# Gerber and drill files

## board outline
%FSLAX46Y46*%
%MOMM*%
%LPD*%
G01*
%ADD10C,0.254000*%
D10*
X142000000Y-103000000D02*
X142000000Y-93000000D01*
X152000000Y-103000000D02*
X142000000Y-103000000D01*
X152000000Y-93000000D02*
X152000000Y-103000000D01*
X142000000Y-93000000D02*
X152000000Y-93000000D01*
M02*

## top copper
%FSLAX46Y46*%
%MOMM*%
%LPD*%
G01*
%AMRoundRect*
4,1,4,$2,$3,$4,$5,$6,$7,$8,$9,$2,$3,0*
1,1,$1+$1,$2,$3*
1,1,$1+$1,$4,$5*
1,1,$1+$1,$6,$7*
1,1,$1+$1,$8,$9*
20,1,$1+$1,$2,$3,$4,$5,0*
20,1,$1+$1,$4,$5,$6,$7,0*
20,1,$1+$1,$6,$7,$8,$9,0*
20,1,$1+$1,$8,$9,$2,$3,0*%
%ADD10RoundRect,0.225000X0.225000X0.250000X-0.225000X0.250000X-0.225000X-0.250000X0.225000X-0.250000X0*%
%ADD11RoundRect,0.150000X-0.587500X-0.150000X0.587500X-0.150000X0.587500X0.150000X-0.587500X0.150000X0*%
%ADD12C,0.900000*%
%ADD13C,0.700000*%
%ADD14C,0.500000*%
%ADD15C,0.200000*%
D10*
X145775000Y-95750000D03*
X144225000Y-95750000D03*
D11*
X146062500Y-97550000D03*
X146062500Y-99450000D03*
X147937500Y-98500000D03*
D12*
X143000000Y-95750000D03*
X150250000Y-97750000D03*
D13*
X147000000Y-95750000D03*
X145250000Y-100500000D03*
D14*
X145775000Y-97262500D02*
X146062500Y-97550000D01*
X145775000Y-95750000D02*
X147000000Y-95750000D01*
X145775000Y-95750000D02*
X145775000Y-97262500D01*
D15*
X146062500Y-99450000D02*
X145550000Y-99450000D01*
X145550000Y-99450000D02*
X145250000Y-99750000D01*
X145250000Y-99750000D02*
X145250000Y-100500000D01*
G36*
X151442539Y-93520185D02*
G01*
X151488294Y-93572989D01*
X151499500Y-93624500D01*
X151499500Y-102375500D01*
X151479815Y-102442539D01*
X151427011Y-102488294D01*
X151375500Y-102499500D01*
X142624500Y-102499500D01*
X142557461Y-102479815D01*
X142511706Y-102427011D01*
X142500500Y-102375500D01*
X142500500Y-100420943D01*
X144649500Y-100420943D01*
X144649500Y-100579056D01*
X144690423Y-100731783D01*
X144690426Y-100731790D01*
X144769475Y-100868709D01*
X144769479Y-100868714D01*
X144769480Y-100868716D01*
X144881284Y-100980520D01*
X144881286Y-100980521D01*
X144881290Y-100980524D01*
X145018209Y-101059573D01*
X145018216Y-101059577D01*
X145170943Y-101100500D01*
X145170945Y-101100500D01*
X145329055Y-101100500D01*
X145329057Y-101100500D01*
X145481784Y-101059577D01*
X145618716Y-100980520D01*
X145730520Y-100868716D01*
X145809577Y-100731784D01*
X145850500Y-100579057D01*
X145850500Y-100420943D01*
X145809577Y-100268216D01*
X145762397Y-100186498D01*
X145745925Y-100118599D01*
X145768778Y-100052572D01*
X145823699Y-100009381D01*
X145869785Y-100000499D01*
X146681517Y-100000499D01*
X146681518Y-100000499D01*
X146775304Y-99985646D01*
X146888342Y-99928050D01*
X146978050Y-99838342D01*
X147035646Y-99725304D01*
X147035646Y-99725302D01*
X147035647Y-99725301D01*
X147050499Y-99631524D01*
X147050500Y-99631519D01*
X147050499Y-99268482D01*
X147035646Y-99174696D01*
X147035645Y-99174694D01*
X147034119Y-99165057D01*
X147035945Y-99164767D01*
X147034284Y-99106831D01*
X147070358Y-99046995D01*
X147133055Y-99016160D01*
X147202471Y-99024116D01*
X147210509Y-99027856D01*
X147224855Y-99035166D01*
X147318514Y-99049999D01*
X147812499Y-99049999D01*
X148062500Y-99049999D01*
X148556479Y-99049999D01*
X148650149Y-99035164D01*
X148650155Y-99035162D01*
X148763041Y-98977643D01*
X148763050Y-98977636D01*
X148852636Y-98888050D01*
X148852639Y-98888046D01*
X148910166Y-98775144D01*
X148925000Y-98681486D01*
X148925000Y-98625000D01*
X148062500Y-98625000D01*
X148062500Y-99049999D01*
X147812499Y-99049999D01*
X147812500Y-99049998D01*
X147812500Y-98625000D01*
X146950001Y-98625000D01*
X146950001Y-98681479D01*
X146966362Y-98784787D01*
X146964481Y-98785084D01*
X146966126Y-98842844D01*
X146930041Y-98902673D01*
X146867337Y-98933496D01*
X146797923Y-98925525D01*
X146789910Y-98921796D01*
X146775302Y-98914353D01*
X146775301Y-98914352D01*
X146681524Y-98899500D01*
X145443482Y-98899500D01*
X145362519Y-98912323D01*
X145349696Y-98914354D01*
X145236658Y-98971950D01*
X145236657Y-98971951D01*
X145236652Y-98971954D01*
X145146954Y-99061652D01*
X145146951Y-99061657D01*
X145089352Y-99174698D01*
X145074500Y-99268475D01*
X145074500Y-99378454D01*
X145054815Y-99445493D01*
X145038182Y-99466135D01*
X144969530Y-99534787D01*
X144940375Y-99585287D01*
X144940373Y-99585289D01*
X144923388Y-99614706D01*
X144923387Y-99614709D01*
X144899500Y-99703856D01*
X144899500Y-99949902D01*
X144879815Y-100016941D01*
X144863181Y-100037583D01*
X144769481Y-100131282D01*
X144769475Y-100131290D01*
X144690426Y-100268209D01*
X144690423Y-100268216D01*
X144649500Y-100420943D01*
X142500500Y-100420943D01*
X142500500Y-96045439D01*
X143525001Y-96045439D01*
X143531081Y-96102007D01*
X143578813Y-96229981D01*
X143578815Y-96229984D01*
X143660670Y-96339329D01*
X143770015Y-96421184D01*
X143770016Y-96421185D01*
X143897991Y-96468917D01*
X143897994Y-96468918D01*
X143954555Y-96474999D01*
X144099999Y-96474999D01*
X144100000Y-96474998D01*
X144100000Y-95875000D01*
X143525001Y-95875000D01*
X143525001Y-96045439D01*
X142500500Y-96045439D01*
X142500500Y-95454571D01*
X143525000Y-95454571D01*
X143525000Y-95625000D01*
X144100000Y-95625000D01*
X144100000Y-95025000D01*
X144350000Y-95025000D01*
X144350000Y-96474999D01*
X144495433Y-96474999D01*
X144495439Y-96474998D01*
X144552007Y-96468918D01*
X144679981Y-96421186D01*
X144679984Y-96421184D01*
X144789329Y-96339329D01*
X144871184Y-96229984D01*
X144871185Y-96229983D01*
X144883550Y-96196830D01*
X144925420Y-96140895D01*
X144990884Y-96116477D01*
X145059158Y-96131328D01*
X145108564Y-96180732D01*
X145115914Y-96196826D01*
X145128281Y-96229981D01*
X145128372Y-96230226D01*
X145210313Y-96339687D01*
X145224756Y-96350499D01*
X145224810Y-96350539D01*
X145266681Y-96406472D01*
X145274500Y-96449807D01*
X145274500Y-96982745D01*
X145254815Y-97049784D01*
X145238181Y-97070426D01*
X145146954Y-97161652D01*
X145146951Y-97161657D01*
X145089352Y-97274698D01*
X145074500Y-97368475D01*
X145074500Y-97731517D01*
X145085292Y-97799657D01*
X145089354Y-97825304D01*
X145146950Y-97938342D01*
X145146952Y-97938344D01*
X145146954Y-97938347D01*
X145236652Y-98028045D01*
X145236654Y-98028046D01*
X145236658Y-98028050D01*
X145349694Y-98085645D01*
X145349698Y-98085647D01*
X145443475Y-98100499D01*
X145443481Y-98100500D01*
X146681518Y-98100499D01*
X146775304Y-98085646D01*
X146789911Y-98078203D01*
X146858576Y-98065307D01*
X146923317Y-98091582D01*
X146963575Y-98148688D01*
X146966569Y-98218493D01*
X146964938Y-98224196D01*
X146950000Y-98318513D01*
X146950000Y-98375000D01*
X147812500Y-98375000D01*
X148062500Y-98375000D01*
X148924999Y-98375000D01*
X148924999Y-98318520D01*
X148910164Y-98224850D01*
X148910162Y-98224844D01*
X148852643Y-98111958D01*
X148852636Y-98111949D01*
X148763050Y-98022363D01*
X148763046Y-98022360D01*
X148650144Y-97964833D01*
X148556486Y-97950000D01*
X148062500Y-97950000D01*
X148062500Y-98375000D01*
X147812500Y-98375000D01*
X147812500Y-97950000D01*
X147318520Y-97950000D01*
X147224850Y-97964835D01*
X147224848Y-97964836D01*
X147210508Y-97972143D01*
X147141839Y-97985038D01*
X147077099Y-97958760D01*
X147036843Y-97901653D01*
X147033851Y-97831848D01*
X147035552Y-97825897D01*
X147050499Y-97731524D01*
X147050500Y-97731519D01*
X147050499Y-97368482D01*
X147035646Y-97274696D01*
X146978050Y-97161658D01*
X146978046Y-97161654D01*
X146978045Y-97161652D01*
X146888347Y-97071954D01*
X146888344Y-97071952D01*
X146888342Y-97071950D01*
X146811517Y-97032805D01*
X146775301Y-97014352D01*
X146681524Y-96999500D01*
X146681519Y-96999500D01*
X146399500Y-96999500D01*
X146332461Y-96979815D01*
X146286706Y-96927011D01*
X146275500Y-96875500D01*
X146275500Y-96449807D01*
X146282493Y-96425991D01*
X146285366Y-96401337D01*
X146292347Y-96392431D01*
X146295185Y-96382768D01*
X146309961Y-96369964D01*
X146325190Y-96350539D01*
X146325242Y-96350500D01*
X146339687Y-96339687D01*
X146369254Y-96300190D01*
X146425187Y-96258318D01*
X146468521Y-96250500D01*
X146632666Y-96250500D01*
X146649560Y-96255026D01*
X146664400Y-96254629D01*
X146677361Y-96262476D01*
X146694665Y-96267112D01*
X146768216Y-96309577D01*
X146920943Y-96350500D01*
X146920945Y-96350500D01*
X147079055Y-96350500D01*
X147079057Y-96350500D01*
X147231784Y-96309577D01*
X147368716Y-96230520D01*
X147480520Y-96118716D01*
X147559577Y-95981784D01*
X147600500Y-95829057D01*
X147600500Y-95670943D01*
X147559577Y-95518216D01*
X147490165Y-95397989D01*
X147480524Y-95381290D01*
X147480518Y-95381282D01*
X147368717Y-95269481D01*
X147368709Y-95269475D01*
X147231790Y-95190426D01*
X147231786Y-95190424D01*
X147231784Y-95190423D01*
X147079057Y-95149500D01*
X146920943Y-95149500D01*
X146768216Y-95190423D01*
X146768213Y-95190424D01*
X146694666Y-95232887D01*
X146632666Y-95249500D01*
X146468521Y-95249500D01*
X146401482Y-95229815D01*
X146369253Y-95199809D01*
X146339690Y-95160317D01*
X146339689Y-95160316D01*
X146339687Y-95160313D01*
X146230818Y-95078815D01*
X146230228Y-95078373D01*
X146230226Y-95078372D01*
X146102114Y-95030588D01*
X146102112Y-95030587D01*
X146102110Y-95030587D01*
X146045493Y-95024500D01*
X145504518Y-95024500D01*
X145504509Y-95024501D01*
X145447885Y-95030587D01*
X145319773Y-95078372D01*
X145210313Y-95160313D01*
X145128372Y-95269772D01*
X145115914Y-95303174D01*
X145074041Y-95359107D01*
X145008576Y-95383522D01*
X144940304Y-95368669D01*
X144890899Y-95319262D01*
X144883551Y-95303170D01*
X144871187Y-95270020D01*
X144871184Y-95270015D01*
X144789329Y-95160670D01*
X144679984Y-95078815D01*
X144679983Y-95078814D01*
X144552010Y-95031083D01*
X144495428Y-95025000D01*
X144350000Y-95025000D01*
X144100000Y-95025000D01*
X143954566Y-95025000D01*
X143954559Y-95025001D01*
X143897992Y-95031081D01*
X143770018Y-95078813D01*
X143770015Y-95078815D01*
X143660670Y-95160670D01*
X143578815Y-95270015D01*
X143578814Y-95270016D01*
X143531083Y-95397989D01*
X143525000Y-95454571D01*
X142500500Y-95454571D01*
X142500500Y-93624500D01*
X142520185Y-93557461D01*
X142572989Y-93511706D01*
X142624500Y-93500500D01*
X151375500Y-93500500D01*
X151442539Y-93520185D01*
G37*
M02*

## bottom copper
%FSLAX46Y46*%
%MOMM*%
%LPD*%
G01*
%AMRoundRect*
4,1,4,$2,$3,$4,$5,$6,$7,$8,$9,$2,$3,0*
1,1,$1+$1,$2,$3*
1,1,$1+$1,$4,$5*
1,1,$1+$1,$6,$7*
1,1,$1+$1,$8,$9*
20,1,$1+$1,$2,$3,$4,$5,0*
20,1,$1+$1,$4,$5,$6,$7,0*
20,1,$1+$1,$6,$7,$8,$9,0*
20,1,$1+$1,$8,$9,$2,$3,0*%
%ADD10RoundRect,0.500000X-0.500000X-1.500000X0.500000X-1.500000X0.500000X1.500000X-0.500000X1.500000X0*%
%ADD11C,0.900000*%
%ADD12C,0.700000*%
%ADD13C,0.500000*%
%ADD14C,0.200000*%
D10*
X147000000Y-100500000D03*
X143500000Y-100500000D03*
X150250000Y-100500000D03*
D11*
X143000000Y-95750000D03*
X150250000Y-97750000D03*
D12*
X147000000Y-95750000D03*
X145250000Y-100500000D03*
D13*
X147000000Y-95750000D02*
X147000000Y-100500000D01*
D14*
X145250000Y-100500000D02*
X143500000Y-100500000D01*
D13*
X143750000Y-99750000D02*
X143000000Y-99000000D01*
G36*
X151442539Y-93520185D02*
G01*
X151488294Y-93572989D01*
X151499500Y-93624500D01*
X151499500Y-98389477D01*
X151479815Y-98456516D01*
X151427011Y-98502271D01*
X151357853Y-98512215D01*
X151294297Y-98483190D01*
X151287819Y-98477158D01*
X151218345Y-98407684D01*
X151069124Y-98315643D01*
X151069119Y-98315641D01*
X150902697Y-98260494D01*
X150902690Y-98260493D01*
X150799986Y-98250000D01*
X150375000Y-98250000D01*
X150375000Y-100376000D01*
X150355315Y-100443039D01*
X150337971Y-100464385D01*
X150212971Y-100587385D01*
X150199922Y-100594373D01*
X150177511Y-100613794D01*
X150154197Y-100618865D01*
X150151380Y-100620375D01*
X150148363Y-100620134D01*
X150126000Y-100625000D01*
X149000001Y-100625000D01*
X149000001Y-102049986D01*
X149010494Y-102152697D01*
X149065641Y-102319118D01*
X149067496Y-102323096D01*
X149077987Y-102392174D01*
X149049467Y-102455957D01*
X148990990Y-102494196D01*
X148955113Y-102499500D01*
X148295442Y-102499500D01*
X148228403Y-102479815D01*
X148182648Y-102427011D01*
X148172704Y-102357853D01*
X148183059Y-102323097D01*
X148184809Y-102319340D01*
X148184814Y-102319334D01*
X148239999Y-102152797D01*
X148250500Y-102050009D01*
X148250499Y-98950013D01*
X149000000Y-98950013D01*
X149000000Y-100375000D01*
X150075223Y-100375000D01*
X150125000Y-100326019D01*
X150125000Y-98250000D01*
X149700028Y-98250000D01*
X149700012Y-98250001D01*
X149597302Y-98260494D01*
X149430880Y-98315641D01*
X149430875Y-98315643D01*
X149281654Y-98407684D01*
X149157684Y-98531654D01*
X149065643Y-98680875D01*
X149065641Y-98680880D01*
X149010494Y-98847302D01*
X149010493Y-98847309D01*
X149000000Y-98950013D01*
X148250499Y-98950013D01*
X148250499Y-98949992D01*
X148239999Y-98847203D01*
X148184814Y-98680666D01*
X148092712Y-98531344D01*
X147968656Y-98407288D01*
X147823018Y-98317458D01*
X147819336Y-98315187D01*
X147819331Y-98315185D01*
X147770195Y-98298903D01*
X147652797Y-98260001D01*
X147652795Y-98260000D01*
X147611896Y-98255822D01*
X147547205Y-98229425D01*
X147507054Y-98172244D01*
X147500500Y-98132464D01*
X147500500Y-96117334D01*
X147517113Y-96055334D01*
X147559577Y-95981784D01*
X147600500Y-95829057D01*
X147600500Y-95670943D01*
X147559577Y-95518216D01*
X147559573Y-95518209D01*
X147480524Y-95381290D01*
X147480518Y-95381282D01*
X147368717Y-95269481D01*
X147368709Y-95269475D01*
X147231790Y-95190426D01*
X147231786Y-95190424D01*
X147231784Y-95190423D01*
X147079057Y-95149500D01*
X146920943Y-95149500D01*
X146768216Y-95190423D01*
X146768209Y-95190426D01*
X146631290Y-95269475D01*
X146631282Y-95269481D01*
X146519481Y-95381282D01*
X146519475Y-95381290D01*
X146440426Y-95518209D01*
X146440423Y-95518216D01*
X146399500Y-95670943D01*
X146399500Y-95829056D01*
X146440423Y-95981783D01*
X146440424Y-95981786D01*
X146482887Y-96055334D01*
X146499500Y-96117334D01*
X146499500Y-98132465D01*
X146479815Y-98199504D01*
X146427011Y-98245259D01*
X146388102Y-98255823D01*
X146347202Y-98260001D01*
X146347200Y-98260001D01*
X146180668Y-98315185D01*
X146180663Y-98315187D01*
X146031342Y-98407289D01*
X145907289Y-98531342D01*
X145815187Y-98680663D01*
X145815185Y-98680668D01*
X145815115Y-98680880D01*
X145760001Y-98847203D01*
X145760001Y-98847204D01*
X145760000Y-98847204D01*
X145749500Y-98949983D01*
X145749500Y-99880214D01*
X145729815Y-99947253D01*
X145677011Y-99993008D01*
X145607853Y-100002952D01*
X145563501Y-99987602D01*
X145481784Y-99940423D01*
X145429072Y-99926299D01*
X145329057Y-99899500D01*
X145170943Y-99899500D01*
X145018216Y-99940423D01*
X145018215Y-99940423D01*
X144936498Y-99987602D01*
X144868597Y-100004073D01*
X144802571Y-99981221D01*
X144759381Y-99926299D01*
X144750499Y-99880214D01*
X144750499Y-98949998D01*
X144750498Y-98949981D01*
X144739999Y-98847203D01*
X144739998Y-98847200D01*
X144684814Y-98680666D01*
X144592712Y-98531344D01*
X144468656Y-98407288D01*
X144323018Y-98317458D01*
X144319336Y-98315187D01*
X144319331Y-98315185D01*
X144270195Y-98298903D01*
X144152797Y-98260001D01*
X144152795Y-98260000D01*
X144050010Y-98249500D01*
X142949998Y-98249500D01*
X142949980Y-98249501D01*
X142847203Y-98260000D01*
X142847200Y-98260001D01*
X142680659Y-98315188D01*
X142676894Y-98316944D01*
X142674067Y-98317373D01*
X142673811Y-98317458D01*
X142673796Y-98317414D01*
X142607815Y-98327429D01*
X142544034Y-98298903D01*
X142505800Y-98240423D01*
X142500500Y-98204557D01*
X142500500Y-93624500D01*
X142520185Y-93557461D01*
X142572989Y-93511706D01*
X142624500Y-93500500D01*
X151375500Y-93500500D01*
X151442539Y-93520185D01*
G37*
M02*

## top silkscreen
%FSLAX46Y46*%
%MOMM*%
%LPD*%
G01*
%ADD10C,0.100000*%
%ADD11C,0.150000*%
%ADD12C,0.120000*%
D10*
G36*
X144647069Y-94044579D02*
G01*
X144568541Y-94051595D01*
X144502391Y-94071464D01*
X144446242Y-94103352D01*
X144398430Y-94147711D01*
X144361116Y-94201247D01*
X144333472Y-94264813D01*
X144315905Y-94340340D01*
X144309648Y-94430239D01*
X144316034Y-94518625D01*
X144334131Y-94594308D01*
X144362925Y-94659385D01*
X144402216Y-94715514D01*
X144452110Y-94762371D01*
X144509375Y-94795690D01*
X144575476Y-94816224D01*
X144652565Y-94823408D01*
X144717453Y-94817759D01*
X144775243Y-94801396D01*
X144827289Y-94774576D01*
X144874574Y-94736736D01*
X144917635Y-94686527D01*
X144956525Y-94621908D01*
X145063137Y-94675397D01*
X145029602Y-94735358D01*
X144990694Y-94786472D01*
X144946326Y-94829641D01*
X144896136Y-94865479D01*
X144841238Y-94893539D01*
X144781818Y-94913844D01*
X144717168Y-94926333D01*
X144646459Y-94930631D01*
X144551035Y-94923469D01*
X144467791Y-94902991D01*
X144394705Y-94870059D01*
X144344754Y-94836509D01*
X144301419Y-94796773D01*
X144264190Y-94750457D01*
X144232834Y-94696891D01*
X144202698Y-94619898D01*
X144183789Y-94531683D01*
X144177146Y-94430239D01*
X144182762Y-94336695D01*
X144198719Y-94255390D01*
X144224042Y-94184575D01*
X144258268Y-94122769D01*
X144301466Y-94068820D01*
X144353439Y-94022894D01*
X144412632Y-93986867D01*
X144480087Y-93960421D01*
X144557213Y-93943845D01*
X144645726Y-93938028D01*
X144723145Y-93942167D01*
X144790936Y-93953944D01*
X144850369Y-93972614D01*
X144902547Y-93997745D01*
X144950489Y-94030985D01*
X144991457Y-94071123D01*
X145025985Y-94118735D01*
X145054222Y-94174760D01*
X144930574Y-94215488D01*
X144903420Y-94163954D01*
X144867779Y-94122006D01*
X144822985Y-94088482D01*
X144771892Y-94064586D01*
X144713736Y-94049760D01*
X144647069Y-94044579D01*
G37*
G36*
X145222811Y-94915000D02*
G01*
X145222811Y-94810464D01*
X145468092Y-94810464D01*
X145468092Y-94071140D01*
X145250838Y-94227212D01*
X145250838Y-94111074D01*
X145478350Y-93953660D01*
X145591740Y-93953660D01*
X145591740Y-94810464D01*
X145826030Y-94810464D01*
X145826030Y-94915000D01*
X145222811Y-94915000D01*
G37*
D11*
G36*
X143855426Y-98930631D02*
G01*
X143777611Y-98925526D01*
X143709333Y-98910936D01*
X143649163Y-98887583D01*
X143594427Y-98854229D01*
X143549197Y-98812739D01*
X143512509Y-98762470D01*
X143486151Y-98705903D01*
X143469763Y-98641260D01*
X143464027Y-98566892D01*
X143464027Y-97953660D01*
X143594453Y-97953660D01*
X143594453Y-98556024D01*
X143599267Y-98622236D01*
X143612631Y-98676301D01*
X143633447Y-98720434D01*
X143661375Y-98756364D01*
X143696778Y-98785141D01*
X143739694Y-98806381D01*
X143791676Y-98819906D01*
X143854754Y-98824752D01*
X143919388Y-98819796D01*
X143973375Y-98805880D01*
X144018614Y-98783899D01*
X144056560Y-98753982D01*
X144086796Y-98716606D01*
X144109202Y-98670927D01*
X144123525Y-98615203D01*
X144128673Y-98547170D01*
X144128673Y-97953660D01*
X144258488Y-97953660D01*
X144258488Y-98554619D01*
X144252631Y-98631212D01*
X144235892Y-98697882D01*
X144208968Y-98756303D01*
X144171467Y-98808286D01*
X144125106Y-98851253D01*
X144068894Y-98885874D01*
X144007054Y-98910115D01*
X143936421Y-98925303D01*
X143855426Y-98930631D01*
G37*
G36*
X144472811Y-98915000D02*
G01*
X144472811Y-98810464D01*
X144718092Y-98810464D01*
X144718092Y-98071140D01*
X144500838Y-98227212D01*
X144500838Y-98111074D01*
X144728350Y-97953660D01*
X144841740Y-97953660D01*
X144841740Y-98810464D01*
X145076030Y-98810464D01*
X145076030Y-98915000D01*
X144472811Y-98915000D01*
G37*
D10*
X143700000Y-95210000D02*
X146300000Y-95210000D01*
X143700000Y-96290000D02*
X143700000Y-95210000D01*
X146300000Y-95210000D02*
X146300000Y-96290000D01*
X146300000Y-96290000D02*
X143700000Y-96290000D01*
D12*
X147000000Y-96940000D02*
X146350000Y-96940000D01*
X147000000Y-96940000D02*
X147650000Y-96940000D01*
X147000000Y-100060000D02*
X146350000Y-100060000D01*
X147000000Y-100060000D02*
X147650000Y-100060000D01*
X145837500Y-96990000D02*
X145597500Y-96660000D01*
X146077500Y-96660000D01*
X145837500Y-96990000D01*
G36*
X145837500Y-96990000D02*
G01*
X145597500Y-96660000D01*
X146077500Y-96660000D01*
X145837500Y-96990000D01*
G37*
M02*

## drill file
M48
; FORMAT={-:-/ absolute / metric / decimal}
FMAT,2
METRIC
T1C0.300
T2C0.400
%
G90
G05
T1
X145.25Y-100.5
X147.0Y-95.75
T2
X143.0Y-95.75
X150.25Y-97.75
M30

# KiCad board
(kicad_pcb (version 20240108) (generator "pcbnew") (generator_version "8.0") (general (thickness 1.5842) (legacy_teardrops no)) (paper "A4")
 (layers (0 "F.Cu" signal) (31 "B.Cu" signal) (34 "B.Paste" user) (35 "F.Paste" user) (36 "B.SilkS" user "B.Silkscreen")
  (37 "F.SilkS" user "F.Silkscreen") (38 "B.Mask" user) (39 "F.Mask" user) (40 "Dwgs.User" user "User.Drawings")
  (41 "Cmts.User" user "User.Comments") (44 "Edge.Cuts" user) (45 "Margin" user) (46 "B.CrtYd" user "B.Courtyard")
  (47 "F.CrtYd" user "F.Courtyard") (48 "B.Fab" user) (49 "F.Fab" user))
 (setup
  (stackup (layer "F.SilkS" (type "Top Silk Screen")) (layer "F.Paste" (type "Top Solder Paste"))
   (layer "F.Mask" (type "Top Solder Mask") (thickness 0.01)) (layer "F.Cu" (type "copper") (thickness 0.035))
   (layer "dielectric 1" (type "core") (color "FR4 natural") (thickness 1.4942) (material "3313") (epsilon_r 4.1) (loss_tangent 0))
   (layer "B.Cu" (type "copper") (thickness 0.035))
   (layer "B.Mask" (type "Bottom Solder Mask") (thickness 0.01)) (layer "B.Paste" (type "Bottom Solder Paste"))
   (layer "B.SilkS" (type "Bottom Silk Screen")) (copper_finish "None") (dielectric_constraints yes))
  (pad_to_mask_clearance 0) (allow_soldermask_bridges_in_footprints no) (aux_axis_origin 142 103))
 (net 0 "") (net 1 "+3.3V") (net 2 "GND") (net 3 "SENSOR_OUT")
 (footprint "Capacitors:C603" (layer "F.Cu") (at 145 95.75 180)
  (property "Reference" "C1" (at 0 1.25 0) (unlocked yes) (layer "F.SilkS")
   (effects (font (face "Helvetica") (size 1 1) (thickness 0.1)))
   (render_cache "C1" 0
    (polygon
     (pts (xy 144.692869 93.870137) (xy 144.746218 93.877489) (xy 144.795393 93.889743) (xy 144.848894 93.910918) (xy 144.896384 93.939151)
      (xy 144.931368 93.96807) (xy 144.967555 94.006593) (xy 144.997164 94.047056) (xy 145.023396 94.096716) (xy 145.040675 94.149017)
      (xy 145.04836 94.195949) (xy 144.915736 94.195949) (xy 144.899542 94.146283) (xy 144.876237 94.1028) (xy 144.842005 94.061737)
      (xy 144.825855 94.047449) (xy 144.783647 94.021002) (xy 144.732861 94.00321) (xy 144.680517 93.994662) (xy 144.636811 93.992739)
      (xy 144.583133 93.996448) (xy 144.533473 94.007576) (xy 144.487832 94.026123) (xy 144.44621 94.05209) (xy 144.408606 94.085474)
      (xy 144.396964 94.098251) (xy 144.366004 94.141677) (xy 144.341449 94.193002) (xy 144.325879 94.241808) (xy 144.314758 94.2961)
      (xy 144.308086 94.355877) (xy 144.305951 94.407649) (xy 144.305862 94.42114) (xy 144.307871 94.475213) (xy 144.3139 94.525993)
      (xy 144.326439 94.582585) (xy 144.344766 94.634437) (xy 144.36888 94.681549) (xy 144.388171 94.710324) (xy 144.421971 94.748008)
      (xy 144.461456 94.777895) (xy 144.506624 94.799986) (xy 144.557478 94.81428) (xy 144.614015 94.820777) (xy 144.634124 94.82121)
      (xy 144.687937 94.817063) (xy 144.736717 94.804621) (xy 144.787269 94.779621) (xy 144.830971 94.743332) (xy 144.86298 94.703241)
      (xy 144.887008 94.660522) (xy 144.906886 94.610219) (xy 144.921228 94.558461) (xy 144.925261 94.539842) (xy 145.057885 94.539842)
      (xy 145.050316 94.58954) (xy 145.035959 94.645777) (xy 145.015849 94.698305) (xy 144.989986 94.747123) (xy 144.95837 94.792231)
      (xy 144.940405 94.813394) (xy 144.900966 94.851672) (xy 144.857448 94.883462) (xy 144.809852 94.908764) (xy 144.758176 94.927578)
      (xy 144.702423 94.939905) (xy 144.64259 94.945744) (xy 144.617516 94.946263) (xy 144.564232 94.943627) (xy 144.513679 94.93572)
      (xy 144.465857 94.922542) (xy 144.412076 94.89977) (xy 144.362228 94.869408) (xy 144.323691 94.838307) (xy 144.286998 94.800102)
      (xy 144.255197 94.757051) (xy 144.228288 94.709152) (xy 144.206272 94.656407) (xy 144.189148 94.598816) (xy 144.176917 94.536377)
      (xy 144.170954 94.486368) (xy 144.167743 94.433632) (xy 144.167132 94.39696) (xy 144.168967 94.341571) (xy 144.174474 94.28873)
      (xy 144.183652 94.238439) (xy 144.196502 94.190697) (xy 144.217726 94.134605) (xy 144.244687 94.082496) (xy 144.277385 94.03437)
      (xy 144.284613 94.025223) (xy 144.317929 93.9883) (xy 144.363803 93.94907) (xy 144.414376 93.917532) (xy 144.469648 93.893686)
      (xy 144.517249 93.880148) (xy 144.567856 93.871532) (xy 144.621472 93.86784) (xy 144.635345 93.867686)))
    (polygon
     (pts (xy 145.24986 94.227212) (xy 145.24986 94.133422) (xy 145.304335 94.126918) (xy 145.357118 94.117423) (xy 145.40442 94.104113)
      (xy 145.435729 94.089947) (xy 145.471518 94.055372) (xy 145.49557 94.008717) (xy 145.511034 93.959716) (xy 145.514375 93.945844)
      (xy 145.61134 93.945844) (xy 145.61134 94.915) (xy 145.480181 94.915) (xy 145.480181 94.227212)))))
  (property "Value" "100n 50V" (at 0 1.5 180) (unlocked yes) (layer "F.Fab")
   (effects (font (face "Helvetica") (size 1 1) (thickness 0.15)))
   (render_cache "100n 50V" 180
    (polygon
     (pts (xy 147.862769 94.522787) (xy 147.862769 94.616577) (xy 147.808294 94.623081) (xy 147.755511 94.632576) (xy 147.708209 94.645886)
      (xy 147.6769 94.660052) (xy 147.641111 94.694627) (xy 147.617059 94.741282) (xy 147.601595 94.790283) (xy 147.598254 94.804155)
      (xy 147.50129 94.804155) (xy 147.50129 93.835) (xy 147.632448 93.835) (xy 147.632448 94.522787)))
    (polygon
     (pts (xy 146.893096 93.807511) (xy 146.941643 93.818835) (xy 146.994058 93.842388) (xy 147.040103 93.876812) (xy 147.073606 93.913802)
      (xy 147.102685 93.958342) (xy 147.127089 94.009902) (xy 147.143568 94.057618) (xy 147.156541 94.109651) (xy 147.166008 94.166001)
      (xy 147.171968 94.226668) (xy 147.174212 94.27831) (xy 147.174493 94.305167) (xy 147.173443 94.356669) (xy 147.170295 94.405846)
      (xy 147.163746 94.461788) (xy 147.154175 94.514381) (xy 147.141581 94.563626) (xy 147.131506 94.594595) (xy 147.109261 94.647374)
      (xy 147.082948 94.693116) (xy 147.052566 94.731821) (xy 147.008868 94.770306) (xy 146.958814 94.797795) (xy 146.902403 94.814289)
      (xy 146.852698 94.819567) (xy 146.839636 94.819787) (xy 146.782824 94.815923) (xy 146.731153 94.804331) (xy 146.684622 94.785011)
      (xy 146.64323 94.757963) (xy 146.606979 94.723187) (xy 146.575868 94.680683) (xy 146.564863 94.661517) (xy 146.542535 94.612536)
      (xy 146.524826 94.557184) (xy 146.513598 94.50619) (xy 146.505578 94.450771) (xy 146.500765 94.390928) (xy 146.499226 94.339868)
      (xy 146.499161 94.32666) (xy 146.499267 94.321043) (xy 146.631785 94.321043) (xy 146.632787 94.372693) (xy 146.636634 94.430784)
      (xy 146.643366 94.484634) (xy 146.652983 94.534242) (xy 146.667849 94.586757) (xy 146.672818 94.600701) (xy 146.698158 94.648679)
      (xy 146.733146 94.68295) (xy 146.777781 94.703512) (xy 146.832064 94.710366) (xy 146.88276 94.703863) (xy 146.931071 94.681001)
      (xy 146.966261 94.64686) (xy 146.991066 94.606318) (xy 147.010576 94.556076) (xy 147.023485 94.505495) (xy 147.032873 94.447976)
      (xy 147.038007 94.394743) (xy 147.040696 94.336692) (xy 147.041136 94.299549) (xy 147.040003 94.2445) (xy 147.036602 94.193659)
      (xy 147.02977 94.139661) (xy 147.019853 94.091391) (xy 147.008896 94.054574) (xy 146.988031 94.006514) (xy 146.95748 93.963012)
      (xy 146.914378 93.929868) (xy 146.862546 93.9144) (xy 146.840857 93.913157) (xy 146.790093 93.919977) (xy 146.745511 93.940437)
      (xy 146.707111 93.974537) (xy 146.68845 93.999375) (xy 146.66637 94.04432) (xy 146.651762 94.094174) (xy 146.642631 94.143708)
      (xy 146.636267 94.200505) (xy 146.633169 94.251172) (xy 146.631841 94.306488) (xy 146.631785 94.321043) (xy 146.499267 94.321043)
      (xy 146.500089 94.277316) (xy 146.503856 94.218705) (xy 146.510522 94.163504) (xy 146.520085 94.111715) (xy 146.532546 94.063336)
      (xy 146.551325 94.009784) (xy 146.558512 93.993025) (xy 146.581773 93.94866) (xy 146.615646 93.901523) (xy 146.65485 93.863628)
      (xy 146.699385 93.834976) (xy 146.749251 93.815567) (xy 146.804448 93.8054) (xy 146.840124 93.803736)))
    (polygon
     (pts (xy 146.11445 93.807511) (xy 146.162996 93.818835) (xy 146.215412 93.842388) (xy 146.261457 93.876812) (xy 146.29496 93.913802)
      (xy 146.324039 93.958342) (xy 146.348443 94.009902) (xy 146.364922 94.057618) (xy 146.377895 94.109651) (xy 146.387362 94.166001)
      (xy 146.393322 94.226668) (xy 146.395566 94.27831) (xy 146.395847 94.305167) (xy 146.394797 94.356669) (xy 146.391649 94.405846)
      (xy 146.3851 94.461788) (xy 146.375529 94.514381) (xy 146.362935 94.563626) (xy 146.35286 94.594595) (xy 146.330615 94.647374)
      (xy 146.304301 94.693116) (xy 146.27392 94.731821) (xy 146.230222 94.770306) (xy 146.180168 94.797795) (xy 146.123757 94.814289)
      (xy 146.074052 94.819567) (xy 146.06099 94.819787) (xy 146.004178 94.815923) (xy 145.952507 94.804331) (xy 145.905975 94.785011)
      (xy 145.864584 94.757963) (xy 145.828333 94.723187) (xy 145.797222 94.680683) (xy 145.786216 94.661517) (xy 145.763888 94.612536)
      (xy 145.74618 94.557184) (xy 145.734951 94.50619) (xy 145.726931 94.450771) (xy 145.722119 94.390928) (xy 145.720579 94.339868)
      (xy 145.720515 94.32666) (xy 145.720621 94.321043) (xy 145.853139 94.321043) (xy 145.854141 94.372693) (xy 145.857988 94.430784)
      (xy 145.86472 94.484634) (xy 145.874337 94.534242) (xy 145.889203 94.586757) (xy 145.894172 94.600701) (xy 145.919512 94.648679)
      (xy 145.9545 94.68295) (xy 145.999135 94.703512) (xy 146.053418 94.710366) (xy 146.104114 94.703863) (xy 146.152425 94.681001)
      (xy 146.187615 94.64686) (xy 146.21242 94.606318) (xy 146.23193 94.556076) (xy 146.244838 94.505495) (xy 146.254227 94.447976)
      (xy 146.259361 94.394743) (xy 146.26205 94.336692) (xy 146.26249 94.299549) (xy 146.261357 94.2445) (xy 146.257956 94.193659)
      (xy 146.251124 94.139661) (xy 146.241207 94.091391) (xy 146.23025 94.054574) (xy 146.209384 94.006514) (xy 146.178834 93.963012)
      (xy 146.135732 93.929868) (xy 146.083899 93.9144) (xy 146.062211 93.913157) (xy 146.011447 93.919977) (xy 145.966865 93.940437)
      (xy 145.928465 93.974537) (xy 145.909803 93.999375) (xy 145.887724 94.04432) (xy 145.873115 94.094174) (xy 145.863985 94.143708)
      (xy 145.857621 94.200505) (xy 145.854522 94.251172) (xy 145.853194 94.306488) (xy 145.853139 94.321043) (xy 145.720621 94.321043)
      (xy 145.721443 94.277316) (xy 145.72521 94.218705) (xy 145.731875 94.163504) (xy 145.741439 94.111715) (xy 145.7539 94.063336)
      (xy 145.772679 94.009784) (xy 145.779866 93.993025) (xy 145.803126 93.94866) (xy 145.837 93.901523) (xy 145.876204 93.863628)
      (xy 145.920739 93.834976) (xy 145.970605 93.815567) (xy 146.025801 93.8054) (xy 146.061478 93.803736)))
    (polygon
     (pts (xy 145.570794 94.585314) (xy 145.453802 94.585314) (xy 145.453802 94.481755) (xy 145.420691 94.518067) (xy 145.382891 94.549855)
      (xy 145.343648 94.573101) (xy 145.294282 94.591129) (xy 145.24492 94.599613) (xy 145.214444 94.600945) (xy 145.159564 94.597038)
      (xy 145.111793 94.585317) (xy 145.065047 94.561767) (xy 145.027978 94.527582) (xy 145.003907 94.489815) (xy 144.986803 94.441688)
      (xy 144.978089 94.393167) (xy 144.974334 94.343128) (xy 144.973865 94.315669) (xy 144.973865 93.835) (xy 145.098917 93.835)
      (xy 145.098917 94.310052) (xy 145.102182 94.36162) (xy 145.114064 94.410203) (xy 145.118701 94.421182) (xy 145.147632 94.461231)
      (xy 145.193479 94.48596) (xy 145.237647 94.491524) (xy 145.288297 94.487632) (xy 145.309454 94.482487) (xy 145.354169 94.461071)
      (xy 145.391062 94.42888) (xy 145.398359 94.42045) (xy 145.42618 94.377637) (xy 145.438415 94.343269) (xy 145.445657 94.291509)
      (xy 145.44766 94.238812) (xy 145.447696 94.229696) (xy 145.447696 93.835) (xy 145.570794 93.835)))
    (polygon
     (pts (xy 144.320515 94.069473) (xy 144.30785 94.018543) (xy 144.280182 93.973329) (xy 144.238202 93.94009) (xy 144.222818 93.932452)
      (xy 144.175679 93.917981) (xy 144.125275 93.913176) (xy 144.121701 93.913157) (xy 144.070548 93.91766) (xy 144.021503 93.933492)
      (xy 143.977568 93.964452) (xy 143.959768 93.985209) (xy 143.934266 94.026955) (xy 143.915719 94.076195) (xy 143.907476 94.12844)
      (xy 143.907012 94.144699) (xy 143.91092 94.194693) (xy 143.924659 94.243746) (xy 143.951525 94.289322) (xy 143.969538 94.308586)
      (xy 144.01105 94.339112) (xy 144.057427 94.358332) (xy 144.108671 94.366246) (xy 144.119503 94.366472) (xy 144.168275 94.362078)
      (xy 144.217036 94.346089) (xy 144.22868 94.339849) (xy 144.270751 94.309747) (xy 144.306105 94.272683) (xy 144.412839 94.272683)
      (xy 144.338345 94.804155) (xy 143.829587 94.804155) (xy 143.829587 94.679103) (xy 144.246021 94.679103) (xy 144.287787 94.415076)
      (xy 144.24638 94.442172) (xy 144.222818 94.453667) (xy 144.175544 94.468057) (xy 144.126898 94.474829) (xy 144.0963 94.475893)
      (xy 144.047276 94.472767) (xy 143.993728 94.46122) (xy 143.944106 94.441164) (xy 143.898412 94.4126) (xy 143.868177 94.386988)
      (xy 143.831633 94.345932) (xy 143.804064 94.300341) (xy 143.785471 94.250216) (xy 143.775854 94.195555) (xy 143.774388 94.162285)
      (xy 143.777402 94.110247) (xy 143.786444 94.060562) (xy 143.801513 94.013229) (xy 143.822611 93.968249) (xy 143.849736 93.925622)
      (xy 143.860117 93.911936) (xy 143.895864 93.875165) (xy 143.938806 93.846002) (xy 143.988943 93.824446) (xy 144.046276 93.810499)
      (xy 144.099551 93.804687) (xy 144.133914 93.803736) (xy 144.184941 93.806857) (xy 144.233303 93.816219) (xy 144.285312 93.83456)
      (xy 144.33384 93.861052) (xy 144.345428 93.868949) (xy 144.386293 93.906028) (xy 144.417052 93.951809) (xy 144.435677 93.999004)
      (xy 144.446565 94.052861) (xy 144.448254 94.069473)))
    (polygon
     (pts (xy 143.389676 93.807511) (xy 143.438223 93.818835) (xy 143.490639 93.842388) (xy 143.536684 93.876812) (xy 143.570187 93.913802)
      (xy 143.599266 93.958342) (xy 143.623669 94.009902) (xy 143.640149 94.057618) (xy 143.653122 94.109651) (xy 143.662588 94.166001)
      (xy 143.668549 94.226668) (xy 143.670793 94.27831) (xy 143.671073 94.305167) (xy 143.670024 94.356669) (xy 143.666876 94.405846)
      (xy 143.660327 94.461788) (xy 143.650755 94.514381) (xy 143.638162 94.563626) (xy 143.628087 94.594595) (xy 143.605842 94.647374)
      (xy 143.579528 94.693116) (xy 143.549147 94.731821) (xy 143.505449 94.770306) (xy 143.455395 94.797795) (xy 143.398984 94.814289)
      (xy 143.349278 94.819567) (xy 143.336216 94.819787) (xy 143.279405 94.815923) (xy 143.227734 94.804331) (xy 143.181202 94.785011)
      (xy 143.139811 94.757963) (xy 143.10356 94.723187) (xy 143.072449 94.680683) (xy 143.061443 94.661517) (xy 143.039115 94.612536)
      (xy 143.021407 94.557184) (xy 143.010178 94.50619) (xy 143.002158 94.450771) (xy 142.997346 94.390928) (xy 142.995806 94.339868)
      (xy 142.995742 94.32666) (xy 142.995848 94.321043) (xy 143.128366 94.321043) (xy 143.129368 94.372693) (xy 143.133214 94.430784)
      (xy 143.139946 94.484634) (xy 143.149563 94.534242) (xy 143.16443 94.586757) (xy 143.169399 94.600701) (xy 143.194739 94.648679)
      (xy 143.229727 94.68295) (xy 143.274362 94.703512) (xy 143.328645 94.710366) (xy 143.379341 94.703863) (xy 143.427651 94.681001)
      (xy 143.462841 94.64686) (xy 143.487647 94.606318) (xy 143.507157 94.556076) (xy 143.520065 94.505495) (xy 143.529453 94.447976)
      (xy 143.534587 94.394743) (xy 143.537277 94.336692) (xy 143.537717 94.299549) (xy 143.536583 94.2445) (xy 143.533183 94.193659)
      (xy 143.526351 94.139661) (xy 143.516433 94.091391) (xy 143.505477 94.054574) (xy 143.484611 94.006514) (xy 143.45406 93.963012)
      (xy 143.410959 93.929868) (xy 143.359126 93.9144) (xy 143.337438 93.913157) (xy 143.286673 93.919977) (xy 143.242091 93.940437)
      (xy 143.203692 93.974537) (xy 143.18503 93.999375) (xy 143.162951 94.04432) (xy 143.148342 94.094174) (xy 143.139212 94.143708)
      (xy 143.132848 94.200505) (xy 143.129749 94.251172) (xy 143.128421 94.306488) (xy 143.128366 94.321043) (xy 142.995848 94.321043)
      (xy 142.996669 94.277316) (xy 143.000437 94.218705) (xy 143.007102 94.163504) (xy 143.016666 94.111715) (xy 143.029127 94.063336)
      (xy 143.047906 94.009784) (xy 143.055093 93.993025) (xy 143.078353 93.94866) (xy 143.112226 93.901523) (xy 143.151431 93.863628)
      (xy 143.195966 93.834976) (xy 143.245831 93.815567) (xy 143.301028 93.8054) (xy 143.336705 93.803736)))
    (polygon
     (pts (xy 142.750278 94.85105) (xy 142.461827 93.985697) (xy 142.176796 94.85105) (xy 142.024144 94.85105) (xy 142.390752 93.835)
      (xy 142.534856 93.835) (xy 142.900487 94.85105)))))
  (fp_line (start 1.3 0.54) (end -1.3 0.54) (stroke (width 0.1) (type default)) (layer "F.SilkS"))
  (fp_line (start 1.3 -0.54) (end 1.3 0.54) (stroke (width 0.1) (type default)) (layer "F.SilkS"))
  (fp_line (start -1.3 0.54) (end -1.3 -0.54) (stroke (width 0.1) (type default)) (layer "F.SilkS"))
  (fp_line (start -1.3 -0.54) (end 1.3 -0.54) (stroke (width 0.1) (type default)) (layer "F.SilkS"))
  (pad "1" smd roundrect (at -0.775 0 180) (size 0.9 0.95) (layers "F.Cu" "F.Paste" "F.Mask") (roundrect_rratio 0.25) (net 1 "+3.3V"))
  (pad "2" smd roundrect (at 0.775 0 180) (size 0.9 0.95) (layers "F.Cu" "F.Paste" "F.Mask") (roundrect_rratio 0.25) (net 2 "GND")))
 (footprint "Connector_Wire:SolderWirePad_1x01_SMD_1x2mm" (layer "F.Cu") (at 147 100.5)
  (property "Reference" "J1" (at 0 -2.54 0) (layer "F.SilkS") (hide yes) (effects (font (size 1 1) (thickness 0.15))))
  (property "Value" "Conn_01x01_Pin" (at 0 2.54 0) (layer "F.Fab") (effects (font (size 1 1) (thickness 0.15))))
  (pad "1" smd roundrect (at 0 0) (size 2 4) (layers "B.Cu" "B.Paste" "B.Mask") (roundrect_rratio 0.25) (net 1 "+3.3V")))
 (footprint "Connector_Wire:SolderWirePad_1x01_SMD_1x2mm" (layer "F.Cu") (at 143.5 100.5)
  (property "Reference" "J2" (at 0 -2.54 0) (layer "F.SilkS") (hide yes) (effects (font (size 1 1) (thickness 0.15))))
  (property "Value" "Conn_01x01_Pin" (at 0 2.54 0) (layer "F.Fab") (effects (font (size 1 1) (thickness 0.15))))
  (pad "1" smd roundrect (at 0 0) (size 2 4) (layers "B.Cu" "B.Paste" "B.Mask") (roundrect_rratio 0.25) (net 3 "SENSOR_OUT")))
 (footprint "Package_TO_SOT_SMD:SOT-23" (layer "F.Cu") (at 147 98.5)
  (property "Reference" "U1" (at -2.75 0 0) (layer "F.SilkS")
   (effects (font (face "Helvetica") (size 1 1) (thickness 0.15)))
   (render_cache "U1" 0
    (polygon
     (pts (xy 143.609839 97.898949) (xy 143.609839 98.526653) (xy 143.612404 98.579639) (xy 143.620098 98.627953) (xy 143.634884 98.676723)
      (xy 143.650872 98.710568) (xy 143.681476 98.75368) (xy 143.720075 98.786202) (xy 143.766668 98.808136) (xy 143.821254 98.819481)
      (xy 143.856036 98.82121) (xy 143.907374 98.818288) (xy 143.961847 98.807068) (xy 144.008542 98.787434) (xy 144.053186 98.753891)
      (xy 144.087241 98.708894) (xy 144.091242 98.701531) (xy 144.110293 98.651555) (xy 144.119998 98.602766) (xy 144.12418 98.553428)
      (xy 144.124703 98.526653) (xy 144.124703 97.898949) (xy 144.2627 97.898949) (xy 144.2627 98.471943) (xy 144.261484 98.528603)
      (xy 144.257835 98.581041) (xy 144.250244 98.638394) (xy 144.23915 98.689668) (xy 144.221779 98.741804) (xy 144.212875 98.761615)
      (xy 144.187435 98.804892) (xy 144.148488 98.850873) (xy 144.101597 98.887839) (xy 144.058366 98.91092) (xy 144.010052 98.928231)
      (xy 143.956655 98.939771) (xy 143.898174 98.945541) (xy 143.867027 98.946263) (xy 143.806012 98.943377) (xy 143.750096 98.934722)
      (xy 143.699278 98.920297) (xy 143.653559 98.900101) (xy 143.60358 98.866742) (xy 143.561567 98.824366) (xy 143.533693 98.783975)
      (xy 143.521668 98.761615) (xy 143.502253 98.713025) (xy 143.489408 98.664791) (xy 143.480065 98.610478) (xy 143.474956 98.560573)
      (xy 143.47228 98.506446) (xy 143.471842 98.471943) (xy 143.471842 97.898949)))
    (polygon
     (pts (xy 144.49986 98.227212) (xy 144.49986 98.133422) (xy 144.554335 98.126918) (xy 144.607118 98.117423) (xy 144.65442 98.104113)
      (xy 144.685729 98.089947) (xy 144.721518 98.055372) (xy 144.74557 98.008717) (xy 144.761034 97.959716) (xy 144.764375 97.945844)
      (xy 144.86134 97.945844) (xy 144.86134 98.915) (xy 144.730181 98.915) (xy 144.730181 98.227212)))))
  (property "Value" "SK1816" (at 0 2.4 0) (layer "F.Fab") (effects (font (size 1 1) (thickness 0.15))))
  (fp_line (start 0 -1.56) (end -0.65 -1.56) (stroke (width 0.12) (type solid)) (layer "F.SilkS"))
  (fp_line (start 0 -1.56) (end 0.65 -1.56) (stroke (width 0.12) (type solid)) (layer "F.SilkS"))
  (fp_line (start 0 1.56) (end -0.65 1.56) (stroke (width 0.12) (type solid)) (layer "F.SilkS"))
  (fp_line (start 0 1.56) (end 0.65 1.56) (stroke (width 0.12) (type solid)) (layer "F.SilkS"))
  (fp_poly
   (pts (xy -1.1625 -1.51) (xy -1.4025 -1.84) (xy -0.9225 -1.84) (xy -1.1625 -1.51)) (stroke (width 0.12) (type solid)) (fill solid)
   (layer "F.SilkS"))
  (pad "1" smd roundrect (at -0.9375 -0.95) (size 1.475 0.6) (layers "F.Cu" "F.Paste" "F.Mask") (roundrect_rratio 0.25) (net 1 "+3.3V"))
  (pad "2" smd roundrect (at -0.9375 0.95) (size 1.475 0.6) (layers "F.Cu" "F.Paste" "F.Mask") (roundrect_rratio 0.25) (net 3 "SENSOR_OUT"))
  (pad "3" smd roundrect (at 0.9375 0) (size 1.475 0.6) (layers "F.Cu" "F.Paste" "F.Mask") (roundrect_rratio 0.25) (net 2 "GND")))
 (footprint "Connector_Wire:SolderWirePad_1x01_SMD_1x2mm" (layer "F.Cu") (at 150.25 100.5)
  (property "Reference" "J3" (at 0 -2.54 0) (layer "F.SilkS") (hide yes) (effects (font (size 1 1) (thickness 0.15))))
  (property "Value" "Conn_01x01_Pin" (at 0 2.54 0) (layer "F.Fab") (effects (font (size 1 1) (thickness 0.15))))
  (pad "1" smd roundrect (at 0 0) (size 2 4) (layers "B.Cu" "B.Paste" "B.Mask") (roundrect_rratio 0.25) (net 2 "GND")))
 (gr_line (start 142 103) (end 142 93) (stroke (width 0.254) (type default)) (layer "Edge.Cuts"))
 (gr_line (start 152 103) (end 142 103) (stroke (width 0.254) (type default)) (layer "Edge.Cuts"))
 (gr_line (start 152 93) (end 152 103) (stroke (width 0.254) (type default)) (layer "Edge.Cuts"))
 (gr_line (start 142 93) (end 152 93) (stroke (width 0.254) (type default)) (layer "Edge.Cuts"))
 (via (at 143 95.75) (size 0.9) (drill 0.4) (layers "F.Cu" "B.Cu") (free yes) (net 2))
 (via (at 150.25 97.75) (size 0.9) (drill 0.4) (layers "F.Cu" "B.Cu") (free yes) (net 2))
 (segment (start 145.775 97.2625) (end 146.0625 97.55) (width 0.5) (layer "F.Cu") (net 1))
 (segment (start 145.775 95.75) (end 147 95.75) (width 0.5) (layer "F.Cu") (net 1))
 (segment (start 145.775 95.75) (end 145.775 97.2625) (width 0.5) (layer "F.Cu") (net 1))
 (via (at 147 95.75) (size 0.7) (drill 0.3) (layers "F.Cu" "B.Cu") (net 1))
 (segment (start 147 95.75) (end 147 100.5) (width 0.5) (layer "B.Cu") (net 1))
 (segment (start 146.0625 99.45) (end 145.55 99.45) (width 0.2) (layer "F.Cu") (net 3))
 (segment (start 145.55 99.45) (end 145.25 99.75) (width 0.2) (layer "F.Cu") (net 3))
 (segment (start 145.25 99.75) (end 145.25 100.5) (width 0.2) (layer "F.Cu") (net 3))
 (via (at 145.25 100.5) (size 0.7) (drill 0.3) (layers "F.Cu" "B.Cu") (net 3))
 (segment (start 145.25 100.5) (end 143.5 100.5) (width 0.2) (layer "B.Cu") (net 3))
 (segment (start 143.75 99.75) (end 143 99) (width 0.5) (layer "B.Cu") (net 3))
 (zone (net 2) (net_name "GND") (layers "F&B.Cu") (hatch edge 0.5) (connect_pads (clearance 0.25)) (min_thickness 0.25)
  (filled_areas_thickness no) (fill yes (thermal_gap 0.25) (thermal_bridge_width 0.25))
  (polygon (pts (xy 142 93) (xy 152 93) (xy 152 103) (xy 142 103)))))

